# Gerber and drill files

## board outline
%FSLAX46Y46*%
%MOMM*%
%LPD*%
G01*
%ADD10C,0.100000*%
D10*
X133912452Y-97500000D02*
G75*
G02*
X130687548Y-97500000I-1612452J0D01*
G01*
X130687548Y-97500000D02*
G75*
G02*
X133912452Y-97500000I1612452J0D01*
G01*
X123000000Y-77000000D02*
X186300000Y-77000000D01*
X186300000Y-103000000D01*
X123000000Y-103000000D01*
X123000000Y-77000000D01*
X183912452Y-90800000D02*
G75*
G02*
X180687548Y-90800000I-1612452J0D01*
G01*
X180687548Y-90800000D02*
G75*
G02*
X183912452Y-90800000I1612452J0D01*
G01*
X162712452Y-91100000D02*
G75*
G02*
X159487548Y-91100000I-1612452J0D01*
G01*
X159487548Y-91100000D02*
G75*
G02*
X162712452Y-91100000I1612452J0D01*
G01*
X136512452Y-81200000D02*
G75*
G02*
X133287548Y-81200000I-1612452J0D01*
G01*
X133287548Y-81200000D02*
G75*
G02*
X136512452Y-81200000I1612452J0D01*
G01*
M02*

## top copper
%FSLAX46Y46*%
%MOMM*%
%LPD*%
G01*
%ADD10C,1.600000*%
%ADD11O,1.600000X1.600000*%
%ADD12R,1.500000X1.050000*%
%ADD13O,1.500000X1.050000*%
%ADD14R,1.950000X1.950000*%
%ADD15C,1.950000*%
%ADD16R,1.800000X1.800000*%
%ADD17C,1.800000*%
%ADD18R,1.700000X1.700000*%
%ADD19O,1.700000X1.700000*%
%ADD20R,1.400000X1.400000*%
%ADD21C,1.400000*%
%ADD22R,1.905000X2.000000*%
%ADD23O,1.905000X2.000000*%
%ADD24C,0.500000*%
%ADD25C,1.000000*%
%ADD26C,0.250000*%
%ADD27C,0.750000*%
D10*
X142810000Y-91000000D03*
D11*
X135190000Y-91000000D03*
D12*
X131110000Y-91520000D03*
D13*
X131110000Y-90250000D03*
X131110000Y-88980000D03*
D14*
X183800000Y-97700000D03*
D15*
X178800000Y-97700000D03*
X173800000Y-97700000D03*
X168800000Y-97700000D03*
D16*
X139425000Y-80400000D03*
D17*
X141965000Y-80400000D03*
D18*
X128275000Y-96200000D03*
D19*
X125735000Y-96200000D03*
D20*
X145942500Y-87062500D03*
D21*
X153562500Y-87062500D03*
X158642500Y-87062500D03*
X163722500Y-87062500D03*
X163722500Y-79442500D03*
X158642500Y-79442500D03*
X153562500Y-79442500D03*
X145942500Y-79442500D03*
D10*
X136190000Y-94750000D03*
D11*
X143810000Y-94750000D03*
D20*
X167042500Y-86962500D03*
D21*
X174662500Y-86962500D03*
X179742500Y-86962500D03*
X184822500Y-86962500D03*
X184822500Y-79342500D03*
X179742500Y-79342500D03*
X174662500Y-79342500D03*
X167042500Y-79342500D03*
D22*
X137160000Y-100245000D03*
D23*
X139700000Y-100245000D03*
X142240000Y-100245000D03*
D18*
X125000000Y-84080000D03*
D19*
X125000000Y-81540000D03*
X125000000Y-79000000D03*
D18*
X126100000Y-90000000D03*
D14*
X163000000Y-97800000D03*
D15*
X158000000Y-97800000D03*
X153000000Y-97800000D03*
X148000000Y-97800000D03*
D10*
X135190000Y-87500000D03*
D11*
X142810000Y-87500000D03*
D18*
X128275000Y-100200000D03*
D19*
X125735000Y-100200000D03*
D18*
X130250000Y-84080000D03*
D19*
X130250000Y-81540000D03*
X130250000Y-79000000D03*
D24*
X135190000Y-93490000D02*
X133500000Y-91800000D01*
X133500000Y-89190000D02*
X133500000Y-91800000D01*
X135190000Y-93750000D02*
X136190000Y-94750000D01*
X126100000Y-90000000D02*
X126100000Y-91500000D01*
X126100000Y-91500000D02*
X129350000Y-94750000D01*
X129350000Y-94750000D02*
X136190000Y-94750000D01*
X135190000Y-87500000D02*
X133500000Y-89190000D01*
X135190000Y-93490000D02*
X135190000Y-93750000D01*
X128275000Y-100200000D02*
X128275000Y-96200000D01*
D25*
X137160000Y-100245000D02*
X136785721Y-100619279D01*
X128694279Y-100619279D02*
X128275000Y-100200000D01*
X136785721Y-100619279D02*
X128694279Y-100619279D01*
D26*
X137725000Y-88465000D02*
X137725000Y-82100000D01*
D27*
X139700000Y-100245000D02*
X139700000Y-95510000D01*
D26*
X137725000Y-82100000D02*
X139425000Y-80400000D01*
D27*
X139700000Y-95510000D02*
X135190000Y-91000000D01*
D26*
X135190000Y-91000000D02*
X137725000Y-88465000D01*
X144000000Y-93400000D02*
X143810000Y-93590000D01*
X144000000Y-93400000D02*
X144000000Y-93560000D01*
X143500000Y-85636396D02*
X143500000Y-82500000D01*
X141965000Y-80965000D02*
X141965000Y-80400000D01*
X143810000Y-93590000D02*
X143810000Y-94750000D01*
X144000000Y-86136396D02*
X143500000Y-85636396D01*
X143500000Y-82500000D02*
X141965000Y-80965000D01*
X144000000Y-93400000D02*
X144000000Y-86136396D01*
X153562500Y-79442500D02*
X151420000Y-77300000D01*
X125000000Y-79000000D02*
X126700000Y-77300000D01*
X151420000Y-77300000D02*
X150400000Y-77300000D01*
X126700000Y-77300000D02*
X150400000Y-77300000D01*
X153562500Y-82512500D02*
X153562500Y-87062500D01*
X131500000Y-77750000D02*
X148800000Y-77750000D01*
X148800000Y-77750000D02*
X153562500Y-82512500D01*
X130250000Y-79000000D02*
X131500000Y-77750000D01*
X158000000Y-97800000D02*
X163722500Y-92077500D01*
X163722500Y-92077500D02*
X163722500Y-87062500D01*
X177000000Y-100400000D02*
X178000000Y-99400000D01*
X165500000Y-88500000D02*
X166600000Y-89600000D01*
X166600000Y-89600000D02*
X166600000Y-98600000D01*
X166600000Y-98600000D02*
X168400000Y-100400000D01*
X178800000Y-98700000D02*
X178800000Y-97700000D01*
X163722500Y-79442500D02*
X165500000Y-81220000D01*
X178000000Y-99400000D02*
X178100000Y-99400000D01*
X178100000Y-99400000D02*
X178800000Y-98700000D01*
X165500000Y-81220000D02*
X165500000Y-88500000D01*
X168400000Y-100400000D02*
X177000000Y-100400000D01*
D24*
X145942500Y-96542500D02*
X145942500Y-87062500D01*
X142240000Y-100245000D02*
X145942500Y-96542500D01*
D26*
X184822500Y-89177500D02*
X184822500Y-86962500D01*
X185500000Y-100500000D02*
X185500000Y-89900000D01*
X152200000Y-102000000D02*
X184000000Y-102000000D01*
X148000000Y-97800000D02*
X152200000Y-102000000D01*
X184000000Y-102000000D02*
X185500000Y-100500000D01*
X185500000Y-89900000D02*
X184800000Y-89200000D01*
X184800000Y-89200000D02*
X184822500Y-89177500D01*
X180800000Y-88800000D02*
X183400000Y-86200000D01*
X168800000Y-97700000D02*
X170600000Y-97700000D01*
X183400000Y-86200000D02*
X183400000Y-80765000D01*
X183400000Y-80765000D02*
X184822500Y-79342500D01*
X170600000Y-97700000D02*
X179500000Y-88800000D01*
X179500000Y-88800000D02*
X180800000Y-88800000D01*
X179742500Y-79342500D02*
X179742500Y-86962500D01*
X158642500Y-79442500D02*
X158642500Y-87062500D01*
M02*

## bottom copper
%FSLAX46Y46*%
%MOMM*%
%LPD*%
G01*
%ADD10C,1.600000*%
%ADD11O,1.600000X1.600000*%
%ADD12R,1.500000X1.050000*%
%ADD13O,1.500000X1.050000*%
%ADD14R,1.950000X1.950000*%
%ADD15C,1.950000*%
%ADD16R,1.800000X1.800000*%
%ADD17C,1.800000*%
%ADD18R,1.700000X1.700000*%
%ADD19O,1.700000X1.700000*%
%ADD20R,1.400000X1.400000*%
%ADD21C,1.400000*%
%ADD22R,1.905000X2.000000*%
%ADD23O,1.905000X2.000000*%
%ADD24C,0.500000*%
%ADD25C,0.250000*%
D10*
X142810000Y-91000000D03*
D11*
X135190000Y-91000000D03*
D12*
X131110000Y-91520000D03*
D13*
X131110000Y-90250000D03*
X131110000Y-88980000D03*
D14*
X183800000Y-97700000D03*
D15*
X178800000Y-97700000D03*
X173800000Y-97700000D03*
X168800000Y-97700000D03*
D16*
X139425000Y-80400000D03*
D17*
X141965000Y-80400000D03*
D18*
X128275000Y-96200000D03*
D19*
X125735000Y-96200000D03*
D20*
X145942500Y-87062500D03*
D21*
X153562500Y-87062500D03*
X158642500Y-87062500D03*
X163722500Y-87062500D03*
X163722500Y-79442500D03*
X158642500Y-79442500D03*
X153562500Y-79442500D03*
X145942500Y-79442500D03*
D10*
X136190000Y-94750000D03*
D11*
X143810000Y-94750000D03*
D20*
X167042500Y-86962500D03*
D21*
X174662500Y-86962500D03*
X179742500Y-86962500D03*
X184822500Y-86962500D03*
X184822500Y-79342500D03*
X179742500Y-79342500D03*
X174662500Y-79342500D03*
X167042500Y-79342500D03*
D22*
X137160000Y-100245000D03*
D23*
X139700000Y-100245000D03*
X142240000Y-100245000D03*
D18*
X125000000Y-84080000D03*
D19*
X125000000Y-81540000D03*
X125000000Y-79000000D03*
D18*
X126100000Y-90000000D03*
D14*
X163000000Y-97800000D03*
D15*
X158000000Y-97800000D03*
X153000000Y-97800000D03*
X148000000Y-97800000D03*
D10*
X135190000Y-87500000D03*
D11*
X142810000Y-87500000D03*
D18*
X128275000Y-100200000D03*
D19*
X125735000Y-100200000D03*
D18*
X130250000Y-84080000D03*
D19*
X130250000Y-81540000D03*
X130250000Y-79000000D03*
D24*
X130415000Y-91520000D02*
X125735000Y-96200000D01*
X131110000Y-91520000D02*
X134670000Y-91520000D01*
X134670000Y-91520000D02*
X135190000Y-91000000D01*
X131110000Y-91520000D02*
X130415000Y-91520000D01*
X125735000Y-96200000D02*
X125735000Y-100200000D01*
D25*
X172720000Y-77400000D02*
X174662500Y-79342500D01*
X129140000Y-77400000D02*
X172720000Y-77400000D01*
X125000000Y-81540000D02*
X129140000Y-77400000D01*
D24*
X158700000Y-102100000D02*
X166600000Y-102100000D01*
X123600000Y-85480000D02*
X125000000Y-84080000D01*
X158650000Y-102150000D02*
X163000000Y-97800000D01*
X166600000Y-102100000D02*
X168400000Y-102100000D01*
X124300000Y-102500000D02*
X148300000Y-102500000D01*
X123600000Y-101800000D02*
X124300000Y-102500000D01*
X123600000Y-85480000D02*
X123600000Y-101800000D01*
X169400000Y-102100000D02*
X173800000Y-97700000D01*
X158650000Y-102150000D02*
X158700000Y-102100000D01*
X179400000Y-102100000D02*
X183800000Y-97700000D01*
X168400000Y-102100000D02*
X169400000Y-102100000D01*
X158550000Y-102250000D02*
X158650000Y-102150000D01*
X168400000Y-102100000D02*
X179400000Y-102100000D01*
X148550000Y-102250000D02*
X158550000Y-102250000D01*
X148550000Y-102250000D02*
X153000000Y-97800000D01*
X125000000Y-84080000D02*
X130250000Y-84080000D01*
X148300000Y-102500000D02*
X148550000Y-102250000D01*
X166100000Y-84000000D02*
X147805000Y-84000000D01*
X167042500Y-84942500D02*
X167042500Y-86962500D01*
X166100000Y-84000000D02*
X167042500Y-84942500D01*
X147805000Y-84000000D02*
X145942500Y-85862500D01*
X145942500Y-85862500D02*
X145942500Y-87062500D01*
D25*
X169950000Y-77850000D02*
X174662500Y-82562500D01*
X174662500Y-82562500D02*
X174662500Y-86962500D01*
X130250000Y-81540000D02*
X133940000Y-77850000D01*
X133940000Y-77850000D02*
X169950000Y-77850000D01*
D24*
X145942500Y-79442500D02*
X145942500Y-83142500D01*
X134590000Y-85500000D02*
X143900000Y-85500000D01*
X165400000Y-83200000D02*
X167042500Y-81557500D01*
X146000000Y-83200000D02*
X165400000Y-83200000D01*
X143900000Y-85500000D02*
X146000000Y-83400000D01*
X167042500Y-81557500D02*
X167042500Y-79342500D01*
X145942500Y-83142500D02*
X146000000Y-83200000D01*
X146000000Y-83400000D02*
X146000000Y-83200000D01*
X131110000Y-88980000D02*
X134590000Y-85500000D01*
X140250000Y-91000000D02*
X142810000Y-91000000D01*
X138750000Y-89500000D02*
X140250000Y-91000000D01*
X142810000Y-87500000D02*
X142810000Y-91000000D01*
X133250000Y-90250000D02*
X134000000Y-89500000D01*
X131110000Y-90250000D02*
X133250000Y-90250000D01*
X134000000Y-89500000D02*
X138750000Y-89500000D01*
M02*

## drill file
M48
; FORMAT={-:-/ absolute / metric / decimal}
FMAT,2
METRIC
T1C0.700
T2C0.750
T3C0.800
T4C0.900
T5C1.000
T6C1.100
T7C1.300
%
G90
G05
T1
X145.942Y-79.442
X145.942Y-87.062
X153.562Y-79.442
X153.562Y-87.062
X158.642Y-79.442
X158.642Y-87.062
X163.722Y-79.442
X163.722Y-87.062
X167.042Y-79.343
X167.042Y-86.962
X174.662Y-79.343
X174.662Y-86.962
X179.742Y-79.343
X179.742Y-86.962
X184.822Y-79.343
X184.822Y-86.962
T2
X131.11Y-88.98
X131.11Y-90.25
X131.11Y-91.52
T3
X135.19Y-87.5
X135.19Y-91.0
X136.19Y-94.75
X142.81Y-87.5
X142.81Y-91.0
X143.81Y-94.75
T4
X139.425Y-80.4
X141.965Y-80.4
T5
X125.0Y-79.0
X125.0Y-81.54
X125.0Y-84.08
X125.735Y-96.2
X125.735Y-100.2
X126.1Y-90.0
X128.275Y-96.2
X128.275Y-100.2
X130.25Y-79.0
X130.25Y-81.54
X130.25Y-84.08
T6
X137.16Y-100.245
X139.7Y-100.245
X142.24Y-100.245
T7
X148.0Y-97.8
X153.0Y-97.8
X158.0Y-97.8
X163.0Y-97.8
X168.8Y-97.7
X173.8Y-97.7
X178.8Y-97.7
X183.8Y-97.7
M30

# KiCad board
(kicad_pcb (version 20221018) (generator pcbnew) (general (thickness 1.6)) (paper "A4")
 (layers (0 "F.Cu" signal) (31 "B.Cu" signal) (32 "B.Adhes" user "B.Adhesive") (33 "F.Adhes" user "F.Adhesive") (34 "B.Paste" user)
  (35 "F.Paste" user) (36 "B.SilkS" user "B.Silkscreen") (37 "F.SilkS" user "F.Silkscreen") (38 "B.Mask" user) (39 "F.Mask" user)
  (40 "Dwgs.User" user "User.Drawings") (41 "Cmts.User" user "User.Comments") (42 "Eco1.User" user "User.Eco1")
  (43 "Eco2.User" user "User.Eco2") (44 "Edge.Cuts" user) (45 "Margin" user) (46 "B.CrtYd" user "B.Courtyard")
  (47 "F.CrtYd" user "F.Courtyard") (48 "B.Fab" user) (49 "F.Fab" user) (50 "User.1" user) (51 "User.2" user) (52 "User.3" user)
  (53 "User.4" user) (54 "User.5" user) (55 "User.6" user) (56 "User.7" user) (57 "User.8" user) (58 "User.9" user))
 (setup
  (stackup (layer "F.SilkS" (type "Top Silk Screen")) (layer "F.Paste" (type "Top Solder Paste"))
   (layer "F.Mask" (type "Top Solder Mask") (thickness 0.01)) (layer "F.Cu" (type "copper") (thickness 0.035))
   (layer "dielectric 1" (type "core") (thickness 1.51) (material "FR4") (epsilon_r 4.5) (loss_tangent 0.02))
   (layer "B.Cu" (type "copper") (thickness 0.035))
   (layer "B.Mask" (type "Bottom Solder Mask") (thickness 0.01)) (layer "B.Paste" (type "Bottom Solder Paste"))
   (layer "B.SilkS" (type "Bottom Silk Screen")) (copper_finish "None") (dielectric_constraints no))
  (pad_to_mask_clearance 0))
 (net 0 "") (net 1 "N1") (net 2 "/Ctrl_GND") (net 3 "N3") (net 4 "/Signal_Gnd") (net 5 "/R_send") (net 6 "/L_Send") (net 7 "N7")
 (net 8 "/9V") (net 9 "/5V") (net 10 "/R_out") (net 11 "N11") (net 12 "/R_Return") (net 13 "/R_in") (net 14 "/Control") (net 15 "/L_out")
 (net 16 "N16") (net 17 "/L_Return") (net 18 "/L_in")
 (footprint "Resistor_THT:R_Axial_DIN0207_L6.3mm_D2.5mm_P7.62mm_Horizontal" (layer "F.Cu") (at 142.81 91 180)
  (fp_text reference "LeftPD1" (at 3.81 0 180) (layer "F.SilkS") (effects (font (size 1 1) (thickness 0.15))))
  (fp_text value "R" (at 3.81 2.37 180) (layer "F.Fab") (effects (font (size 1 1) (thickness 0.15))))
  (pad "1" thru_hole circle (at 0 0 180) (size 1.6 1.6) (drill 0.8) (layers "*.Cu" "*.Mask") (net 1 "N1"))
  (pad "2" thru_hole oval (at 7.62 0 180) (size 1.6 1.6) (drill 0.8) (layers "*.Cu" "*.Mask") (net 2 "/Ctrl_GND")))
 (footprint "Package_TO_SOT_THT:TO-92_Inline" (layer "F.Cu") (at 131.11 91.52 90)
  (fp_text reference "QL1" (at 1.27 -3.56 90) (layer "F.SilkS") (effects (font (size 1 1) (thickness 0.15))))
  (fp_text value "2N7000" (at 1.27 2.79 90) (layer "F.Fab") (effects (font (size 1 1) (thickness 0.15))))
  (pad "1" thru_hole rect (at 0 0 90) (size 1.05 1.5) (drill 0.75) (layers "*.Cu" "*.Mask") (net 2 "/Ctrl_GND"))
  (pad "2" thru_hole oval (at 1.27 0 90) (size 1.05 1.5) (drill 0.75) (layers "*.Cu" "*.Mask") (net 1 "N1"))
  (pad "3" thru_hole oval (at 2.54 0 90) (size 1.05 1.5) (drill 0.75) (layers "*.Cu" "*.Mask") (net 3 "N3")))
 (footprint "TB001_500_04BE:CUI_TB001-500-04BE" (layer "F.Cu") (at 183.8 97.7 180)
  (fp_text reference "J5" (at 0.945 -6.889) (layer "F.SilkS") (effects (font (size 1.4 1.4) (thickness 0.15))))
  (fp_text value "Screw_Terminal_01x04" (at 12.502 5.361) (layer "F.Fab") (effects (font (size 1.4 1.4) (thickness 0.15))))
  (pad "1" thru_hole rect (at 0 0 180) (size 1.95 1.95) (drill 1.3) (layers "*.Cu" "*.Mask") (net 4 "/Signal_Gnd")
   (solder_mask_margin 0.102))
  (pad "2" thru_hole circle (at 5 0 180) (size 1.95 1.95) (drill 1.3) (layers "*.Cu" "*.Mask") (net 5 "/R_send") (solder_mask_margin 0.102))
  (pad "3" thru_hole circle (at 10 0 180) (size 1.95 1.95) (drill 1.3) (layers "*.Cu" "*.Mask") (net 4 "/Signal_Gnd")
   (solder_mask_margin 0.102))
  (pad "4" thru_hole circle (at 15 0 180) (size 1.95 1.95) (drill 1.3) (layers "*.Cu" "*.Mask") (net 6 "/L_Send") (solder_mask_margin 0.102)))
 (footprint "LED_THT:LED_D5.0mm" (layer "F.Cu") (at 139.425 80.4)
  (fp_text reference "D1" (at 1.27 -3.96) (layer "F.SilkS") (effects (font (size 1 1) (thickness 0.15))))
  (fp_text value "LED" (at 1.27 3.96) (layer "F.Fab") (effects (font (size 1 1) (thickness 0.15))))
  (pad "1" thru_hole rect (at 0 0) (size 1.8 1.8) (drill 0.9) (layers "*.Cu" "*.Mask") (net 2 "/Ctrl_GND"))
  (pad "2" thru_hole circle (at 2.54 0) (size 1.8 1.8) (drill 0.9) (layers "*.Cu" "*.Mask") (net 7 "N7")))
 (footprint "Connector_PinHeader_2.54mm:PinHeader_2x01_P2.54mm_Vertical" (layer "F.Cu") (at 128.275 96.2 180)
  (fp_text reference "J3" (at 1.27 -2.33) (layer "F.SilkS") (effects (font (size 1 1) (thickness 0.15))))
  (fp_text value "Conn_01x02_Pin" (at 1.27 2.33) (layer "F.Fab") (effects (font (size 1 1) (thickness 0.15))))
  (pad "1" thru_hole rect (at 0 0 180) (size 1.7 1.7) (drill 1) (layers "*.Cu" "*.Mask") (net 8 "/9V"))
  (pad "2" thru_hole oval (at 2.54 0 180) (size 1.7 1.7) (drill 1) (layers "*.Cu" "*.Mask") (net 2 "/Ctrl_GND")))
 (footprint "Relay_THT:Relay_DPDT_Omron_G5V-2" (layer "F.Cu") (at 145.9425 87.0625 90)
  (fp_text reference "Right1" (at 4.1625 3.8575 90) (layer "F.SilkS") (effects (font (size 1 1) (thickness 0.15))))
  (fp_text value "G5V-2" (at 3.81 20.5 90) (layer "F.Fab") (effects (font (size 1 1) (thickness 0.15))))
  (pad "1" thru_hole rect (at 0 0 90) (size 1.4 1.4) (drill 0.7) (layers "*.Cu" "*.Mask") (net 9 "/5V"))
  (pad "4" thru_hole circle (at 0 7.62 90) (size 1.4 1.4) (drill 0.7) (layers "*.Cu" "*.Mask") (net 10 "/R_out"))
  (pad "6" thru_hole circle (at 0 12.7 90) (size 1.4 1.4) (drill 0.7) (layers "*.Cu" "*.Mask") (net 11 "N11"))
  (pad "8" thru_hole circle (at 0 17.78 90) (size 1.4 1.4) (drill 0.7) (layers "*.Cu" "*.Mask") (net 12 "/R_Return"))
  (pad "9" thru_hole circle (at 7.62 17.78 90) (size 1.4 1.4) (drill 0.7) (layers "*.Cu" "*.Mask") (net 5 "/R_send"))
  (pad "11" thru_hole circle (at 7.62 12.7 90) (size 1.4 1.4) (drill 0.7) (layers "*.Cu" "*.Mask") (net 11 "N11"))
  (pad "13" thru_hole circle (at 7.62 7.62 90) (size 1.4 1.4) (drill 0.7) (layers "*.Cu" "*.Mask") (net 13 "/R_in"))
  (pad "16" thru_hole circle (at 7.62 0 90) (size 1.4 1.4) (drill 0.7) (layers "*.Cu" "*.Mask") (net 3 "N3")))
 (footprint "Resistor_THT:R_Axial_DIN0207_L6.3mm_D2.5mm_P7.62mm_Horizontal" (layer "F.Cu") (at 136.19 94.75)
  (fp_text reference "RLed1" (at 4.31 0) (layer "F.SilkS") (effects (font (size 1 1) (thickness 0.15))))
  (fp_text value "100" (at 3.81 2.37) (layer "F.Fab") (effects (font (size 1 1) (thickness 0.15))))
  (pad "1" thru_hole circle (at 0 0) (size 1.6 1.6) (drill 0.8) (layers "*.Cu" "*.Mask") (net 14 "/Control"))
  (pad "2" thru_hole oval (at 7.62 0) (size 1.6 1.6) (drill 0.8) (layers "*.Cu" "*.Mask") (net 7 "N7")))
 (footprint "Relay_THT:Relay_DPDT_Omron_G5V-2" (layer "F.Cu") (at 167.0425 86.9625 90)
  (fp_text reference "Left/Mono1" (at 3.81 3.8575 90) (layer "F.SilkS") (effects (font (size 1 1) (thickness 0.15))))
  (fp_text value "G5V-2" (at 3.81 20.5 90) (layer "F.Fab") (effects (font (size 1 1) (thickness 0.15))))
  (pad "1" thru_hole rect (at 0 0 90) (size 1.4 1.4) (drill 0.7) (layers "*.Cu" "*.Mask") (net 9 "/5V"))
  (pad "4" thru_hole circle (at 0 7.62 90) (size 1.4 1.4) (drill 0.7) (layers "*.Cu" "*.Mask") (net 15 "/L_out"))
  (pad "6" thru_hole circle (at 0 12.7 90) (size 1.4 1.4) (drill 0.7) (layers "*.Cu" "*.Mask") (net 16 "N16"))
  (pad "8" thru_hole circle (at 0 17.78 90) (size 1.4 1.4) (drill 0.7) (layers "*.Cu" "*.Mask") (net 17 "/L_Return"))
  (pad "9" thru_hole circle (at 7.62 17.78 90) (size 1.4 1.4) (drill 0.7) (layers "*.Cu" "*.Mask") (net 6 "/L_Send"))
  (pad "11" thru_hole circle (at 7.62 12.7 90) (size 1.4 1.4) (drill 0.7) (layers "*.Cu" "*.Mask") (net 16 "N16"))
  (pad "13" thru_hole circle (at 7.62 7.62 90) (size 1.4 1.4) (drill 0.7) (layers "*.Cu" "*.Mask") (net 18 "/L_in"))
  (pad "16" thru_hole circle (at 7.62 0 90) (size 1.4 1.4) (drill 0.7) (layers "*.Cu" "*.Mask") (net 3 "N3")))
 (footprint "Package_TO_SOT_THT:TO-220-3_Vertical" (layer "F.Cu") (at 137.16 100.245)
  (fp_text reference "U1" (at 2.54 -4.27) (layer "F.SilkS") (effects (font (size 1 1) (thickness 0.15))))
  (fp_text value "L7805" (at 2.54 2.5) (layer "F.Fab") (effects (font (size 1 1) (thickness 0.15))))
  (pad "1" thru_hole rect (at 0 0) (size 1.905 2) (drill 1.1) (layers "*.Cu" "*.Mask") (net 8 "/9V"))
  (pad "2" thru_hole oval (at 2.54 0) (size 1.905 2) (drill 1.1) (layers "*.Cu" "*.Mask") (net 2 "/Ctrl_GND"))
  (pad "3" thru_hole oval (at 5.08 0) (size 1.905 2) (drill 1.1) (layers "*.Cu" "*.Mask") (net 9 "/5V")))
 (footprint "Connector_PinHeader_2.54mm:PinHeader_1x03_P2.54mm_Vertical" (layer "F.Cu") (at 125 84.08 180)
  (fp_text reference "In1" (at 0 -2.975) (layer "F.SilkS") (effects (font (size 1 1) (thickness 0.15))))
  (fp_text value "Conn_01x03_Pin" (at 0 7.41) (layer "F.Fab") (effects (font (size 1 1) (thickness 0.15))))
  (pad "1" thru_hole rect (at 0 0 180) (size 1.7 1.7) (drill 1) (layers "*.Cu" "*.Mask") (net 4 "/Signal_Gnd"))
  (pad "2" thru_hole oval (at 0 2.54 180) (size 1.7 1.7) (drill 1) (layers "*.Cu" "*.Mask") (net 18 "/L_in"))
  (pad "3" thru_hole oval (at 0 5.08 180) (size 1.7 1.7) (drill 1) (layers "*.Cu" "*.Mask") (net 13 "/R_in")))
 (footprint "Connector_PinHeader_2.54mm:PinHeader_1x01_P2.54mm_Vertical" (layer "F.Cu") (at 126.1 90 90)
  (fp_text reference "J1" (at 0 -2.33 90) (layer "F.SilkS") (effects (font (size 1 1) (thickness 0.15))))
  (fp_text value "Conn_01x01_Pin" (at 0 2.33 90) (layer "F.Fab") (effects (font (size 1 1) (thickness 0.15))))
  (pad "1" thru_hole rect (at 0 0 90) (size 1.7 1.7) (drill 1) (layers "*.Cu" "*.Mask") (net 14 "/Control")))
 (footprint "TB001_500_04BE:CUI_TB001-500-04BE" (layer "F.Cu") (at 163 97.8 180)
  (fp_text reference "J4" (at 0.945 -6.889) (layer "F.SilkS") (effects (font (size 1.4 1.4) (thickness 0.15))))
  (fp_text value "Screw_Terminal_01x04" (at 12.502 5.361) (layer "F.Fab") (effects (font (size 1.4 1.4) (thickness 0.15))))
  (pad "1" thru_hole rect (at 0 0 180) (size 1.95 1.95) (drill 1.3) (layers "*.Cu" "*.Mask") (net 4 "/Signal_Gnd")
   (solder_mask_margin 0.102))
  (pad "2" thru_hole circle (at 5 0 180) (size 1.95 1.95) (drill 1.3) (layers "*.Cu" "*.Mask") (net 12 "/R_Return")
   (solder_mask_margin 0.102))
  (pad "3" thru_hole circle (at 10 0 180) (size 1.95 1.95) (drill 1.3) (layers "*.Cu" "*.Mask") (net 4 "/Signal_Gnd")
   (solder_mask_margin 0.102))
  (pad "4" thru_hole circle (at 15 0 180) (size 1.95 1.95) (drill 1.3) (layers "*.Cu" "*.Mask") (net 17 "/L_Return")
   (solder_mask_margin 0.102)))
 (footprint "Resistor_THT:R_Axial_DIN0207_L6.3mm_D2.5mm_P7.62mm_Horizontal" (layer "F.Cu") (at 135.19 87.5)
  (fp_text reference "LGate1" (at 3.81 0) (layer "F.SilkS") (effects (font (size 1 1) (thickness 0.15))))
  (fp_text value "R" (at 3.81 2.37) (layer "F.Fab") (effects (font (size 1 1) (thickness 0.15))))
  (pad "1" thru_hole circle (at 0 0) (size 1.6 1.6) (drill 0.8) (layers "*.Cu" "*.Mask") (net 14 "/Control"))
  (pad "2" thru_hole oval (at 7.62 0) (size 1.6 1.6) (drill 0.8) (layers "*.Cu" "*.Mask") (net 1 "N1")))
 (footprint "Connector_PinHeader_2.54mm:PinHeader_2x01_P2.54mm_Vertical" (layer "F.Cu") (at 128.275 100.2 180)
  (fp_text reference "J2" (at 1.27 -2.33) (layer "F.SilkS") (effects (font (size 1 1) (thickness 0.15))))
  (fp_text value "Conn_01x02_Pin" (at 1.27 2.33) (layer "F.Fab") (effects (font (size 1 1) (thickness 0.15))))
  (pad "1" thru_hole rect (at 0 0 180) (size 1.7 1.7) (drill 1) (layers "*.Cu" "*.Mask") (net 8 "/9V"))
  (pad "2" thru_hole oval (at 2.54 0 180) (size 1.7 1.7) (drill 1) (layers "*.Cu" "*.Mask") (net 2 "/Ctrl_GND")))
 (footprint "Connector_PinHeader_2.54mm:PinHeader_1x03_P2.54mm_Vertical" (layer "F.Cu") (at 130.25 84.08 180)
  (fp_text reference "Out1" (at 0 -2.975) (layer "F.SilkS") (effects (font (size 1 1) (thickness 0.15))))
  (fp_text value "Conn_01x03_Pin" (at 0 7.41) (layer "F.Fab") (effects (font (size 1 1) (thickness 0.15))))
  (pad "1" thru_hole rect (at 0 0 180) (size 1.7 1.7) (drill 1) (layers "*.Cu" "*.Mask") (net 4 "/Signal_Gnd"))
  (pad "2" thru_hole oval (at 0 2.54 180) (size 1.7 1.7) (drill 1) (layers "*.Cu" "*.Mask") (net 15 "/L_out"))
  (pad "3" thru_hole oval (at 0 5.08 180) (size 1.7 1.7) (drill 1) (layers "*.Cu" "*.Mask") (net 10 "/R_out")))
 (gr_circle (center 132.3 97.5) (end 132.1 95.9) (stroke (width 0.1) (type default)) (fill none) (layer "Edge.Cuts"))
 (gr_rect (start 123 77) (end 186.3 103) (stroke (width 0.1) (type default)) (fill none) (layer "Edge.Cuts"))
 (gr_circle (center 182.3 90.8) (end 182.1 89.2) (stroke (width 0.1) (type default)) (fill none) (layer "Edge.Cuts"))
 (gr_circle (center 161.1 91.1) (end 160.9 89.5) (stroke (width 0.1) (type default)) (fill none) (layer "Edge.Cuts"))
 (gr_circle (center 134.9 81.2) (end 134.7 79.6) (stroke (width 0.1) (type default)) (fill none) (layer "Edge.Cuts"))
 (segment (start 135.19 93.49) (end 133.5 91.8) (width 0.5) (layer "F.Cu") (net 14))
 (segment (start 133.5 89.19) (end 133.5 91.8) (width 0.5) (layer "F.Cu") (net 14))
 (segment (start 135.19 93.75) (end 136.19 94.75) (width 0.5) (layer "F.Cu") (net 14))
 (segment (start 126.1 90) (end 126.1 91.5) (width 0.5) (layer "F.Cu") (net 14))
 (segment (start 126.1 91.5) (end 129.35 94.75) (width 0.5) (layer "F.Cu") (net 14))
 (segment (start 129.35 94.75) (end 136.19 94.75) (width 0.5) (layer "F.Cu") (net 14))
 (segment (start 135.19 87.5) (end 133.5 89.19) (width 0.5) (layer "F.Cu") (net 14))
 (segment (start 135.19 93.49) (end 135.19 93.75) (width 0.5) (layer "F.Cu") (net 14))
 (segment (start 128.275 100.2) (end 128.275 96.2) (width 0.5) (layer "F.Cu") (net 8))
 (segment (start 137.16 100.245) (end 136.785721 100.619279) (width 1) (layer "F.Cu") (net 8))
 (segment (start 128.694279 100.619279) (end 128.275 100.2) (width 1) (layer "F.Cu") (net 8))
 (segment (start 136.785721 100.619279) (end 128.694279 100.619279) (width 1) (layer "F.Cu") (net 8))
 (segment (start 137.725 88.465) (end 137.725 82.1) (width 0.25) (layer "F.Cu") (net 2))
 (segment (start 139.7 100.245) (end 139.7 95.51) (width 0.75) (layer "F.Cu") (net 2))
 (segment (start 137.725 82.1) (end 139.425 80.4) (width 0.25) (layer "F.Cu") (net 2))
 (segment (start 139.7 95.51) (end 135.19 91) (width 0.75) (layer "F.Cu") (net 2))
 (segment (start 135.19 91) (end 137.725 88.465) (width 0.25) (layer "F.Cu") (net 2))
 (segment (start 130.415 91.52) (end 125.735 96.2) (width 0.5) (layer "B.Cu") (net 2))
 (segment (start 131.11 91.52) (end 134.67 91.52) (width 0.5) (layer "B.Cu") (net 2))
 (segment (start 134.67 91.52) (end 135.19 91) (width 0.5) (layer "B.Cu") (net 2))
 (segment (start 131.11 91.52) (end 130.415 91.52) (width 0.5) (layer "B.Cu") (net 2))
 (segment (start 125.735 96.2) (end 125.735 100.2) (width 0.5) (layer "B.Cu") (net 2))
 (segment (start 144 93.4) (end 143.81 93.59) (width 0.25) (layer "F.Cu") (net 7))
 (segment (start 144 93.4) (end 144 93.56) (width 0.25) (layer "F.Cu") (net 7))
 (segment (start 143.5 85.636396) (end 143.5 82.5) (width 0.25) (layer "F.Cu") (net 7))
 (segment (start 141.965 80.965) (end 141.965 80.4) (width 0.25) (layer "F.Cu") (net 7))
 (segment (start 143.81 93.59) (end 143.81 94.75) (width 0.25) (layer "F.Cu") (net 7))
 (segment (start 144 86.136396) (end 143.5 85.636396) (width 0.25) (layer "F.Cu") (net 7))
 (segment (start 143.5 82.5) (end 141.965 80.965) (width 0.25) (layer "F.Cu") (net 7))
 (segment (start 144 93.4) (end 144 86.136396) (width 0.25) (layer "F.Cu") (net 7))
 (segment (start 153.5625 79.4425) (end 151.42 77.3) (width 0.25) (layer "F.Cu") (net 13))
 (segment (start 125 79) (end 126.7 77.3) (width 0.25) (layer "F.Cu") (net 13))
 (segment (start 151.42 77.3) (end 150.4 77.3) (width 0.25) (layer "F.Cu") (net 13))
 (segment (start 126.7 77.3) (end 150.4 77.3) (width 0.25) (layer "F.Cu") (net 13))
 (segment (start 172.72 77.4) (end 174.6625 79.3425) (width 0.25) (layer "B.Cu") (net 18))
 (segment (start 129.14 77.4) (end 172.72 77.4) (width 0.25) (layer "B.Cu") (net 18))
 (segment (start 125 81.54) (end 129.14 77.4) (width 0.25) (layer "B.Cu") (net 18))
 (segment (start 158.7 102.1) (end 166.6 102.1) (width 0.5) (layer "B.Cu") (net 4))
 (segment (start 123.6 85.48) (end 125 84.08) (width 0.5) (layer "B.Cu") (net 4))
 (segment (start 158.65 102.15) (end 163 97.8) (width 0.5) (layer "B.Cu") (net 4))
 (segment (start 166.6 102.1) (end 168.4 102.1) (width 0.5) (layer "B.Cu") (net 4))
 (segment (start 124.3 102.5) (end 148.3 102.5) (width 0.5) (layer "B.Cu") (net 4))
 (segment (start 123.6 101.8) (end 124.3 102.5) (width 0.5) (layer "B.Cu") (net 4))
 (segment (start 123.6 85.48) (end 123.6 101.8) (width 0.5) (layer "B.Cu") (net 4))
 (segment (start 169.4 102.1) (end 173.8 97.7) (width 0.5) (layer "B.Cu") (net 4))
 (segment (start 158.65 102.15) (end 158.7 102.1) (width 0.5) (layer "B.Cu") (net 4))
 (segment (start 179.4 102.1) (end 183.8 97.7) (width 0.5) (layer "B.Cu") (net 4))
 (segment (start 168.4 102.1) (end 169.4 102.1) (width 0.5) (layer "B.Cu") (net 4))
 (segment (start 158.55 102.25) (end 158.65 102.15) (width 0.5) (layer "B.Cu") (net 4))
 (segment (start 168.4 102.1) (end 179.4 102.1) (width 0.5) (layer "B.Cu") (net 4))
 (segment (start 148.55 102.25) (end 158.55 102.25) (width 0.5) (layer "B.Cu") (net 4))
 (segment (start 148.55 102.25) (end 153 97.8) (width 0.5) (layer "B.Cu") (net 4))
 (segment (start 125 84.08) (end 130.25 84.08) (width 0.5) (layer "B.Cu") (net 4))
 (segment (start 148.3 102.5) (end 148.55 102.25) (width 0.5) (layer "B.Cu") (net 4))
 (segment (start 153.5625 82.5125) (end 153.5625 87.0625) (width 0.25) (layer "F.Cu") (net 10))
 (segment (start 131.5 77.75) (end 148.8 77.75) (width 0.25) (layer "F.Cu") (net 10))
 (segment (start 148.8 77.75) (end 153.5625 82.5125) (width 0.25) (layer "F.Cu") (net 10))
 (segment (start 130.25 79) (end 131.5 77.75) (width 0.25) (layer "F.Cu") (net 10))
 (segment (start 158 97.8) (end 163.7225 92.0775) (width 0.25) (layer "F.Cu") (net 12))
 (segment (start 163.7225 92.0775) (end 163.7225 87.0625) (width 0.25) (layer "F.Cu") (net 12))
 (segment (start 177 100.4) (end 178 99.4) (width 0.25) (layer "F.Cu") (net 5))
 (segment (start 165.5 88.5) (end 166.6 89.6) (width 0.25) (layer "F.Cu") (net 5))
 (segment (start 166.6 89.6) (end 166.6 98.6) (width 0.25) (layer "F.Cu") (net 5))
 (segment (start 166.6 98.6) (end 168.4 100.4) (width 0.25) (layer "F.Cu") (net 5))
 (segment (start 178.8 98.7) (end 178.8 97.7) (width 0.25) (layer "F.Cu") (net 5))
 (segment (start 163.7225 79.4425) (end 165.5 81.22) (width 0.25) (layer "F.Cu") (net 5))
 (segment (start 178 99.4) (end 178.1 99.4) (width 0.25) (layer "F.Cu") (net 5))
 (segment (start 178.1 99.4) (end 178.8 98.7) (width 0.25) (layer "F.Cu") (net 5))
 (segment (start 165.5 81.22) (end 165.5 88.5) (width 0.25) (layer "F.Cu") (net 5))
 (segment (start 168.4 100.4) (end 177 100.4) (width 0.25) (layer "F.Cu") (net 5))
 (segment (start 145.9425 96.5425) (end 145.9425 87.0625) (width 0.5) (layer "F.Cu") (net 9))
 (segment (start 142.24 100.245) (end 145.9425 96.5425) (width 0.5) (layer "F.Cu") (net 9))
 (segment (start 166.1 84) (end 147.805 84) (width 0.5) (layer "B.Cu") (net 9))
 (segment (start 167.0425 84.9425) (end 167.0425 86.9625) (width 0.5) (layer "B.Cu") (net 9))
 (segment (start 166.1 84) (end 167.0425 84.9425) (width 0.5) (layer "B.Cu") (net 9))
 (segment (start 147.805 84) (end 145.9425 85.8625) (width 0.5) (layer "B.Cu") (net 9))
 (segment (start 145.9425 85.8625) (end 145.9425 87.0625) (width 0.5) (layer "B.Cu") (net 9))
 (segment (start 169.95 77.85) (end 174.6625 82.5625) (width 0.25) (layer "B.Cu") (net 15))
 (segment (start 174.6625 82.5625) (end 174.6625 86.9625) (width 0.25) (layer "B.Cu") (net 15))
 (segment (start 130.25 81.54) (end 133.94 77.85) (width 0.25) (layer "B.Cu") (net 15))
 (segment (start 133.94 77.85) (end 169.95 77.85) (width 0.25) (layer "B.Cu") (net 15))
 (segment (start 184.8225 89.1775) (end 184.8225 86.9625) (width 0.25) (layer "F.Cu") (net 17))
 (segment (start 185.5 100.5) (end 185.5 89.9) (width 0.25) (layer "F.Cu") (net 17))
 (segment (start 152.2 102) (end 184 102) (width 0.25) (layer "F.Cu") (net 17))
 (segment (start 148 97.8) (end 152.2 102) (width 0.25) (layer "F.Cu") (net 17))
 (segment (start 184 102) (end 185.5 100.5) (width 0.25) (layer "F.Cu") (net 17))
 (segment (start 185.5 89.9) (end 184.8 89.2) (width 0.25) (layer "F.Cu") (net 17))
 (segment (start 184.8 89.2) (end 184.8225 89.1775) (width 0.25) (layer "F.Cu") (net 17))
 (segment (start 180.8 88.8) (end 183.4 86.2) (width 0.25) (layer "F.Cu") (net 6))
 (segment (start 168.8 97.7) (end 170.6 97.7) (width 0.25) (layer "F.Cu") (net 6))
 (segment (start 183.4 86.2) (end 183.4 80.765) (width 0.25) (layer "F.Cu") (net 6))
 (segment (start 183.4 80.765) (end 184.8225 79.3425) (width 0.25) (layer "F.Cu") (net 6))
 (segment (start 170.6 97.7) (end 179.5 88.8) (width 0.25) (layer "F.Cu") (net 6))
 (segment (start 179.5 88.8) (end 180.8 88.8) (width 0.25) (layer "F.Cu") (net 6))
 (segment (start 179.7425 79.3425) (end 179.7425 86.9625) (width 0.25) (layer "F.Cu") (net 16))
 (segment (start 158.6425 79.4425) (end 158.6425 87.0625) (width 0.25) (layer "F.Cu") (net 11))
 (segment (start 145.9425 79.4425) (end 145.9425 83.1425) (width 0.5) (layer "B.Cu") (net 3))
 (segment (start 134.59 85.5) (end 143.9 85.5) (width 0.5) (layer "B.Cu") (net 3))
 (segment (start 165.4 83.2) (end 167.0425 81.5575) (width 0.5) (layer "B.Cu") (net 3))
 (segment (start 146 83.2) (end 165.4 83.2) (width 0.5) (layer "B.Cu") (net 3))
 (segment (start 143.9 85.5) (end 146 83.4) (width 0.5) (layer "B.Cu") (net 3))
 (segment (start 167.0425 81.5575) (end 167.0425 79.3425) (width 0.5) (layer "B.Cu") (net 3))
 (segment (start 145.9425 83.1425) (end 146 83.2) (width 0.5) (layer "B.Cu") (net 3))
 (segment (start 146 83.4) (end 146 83.2) (width 0.5) (layer "B.Cu") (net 3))
 (segment (start 131.11 88.98) (end 134.59 85.5) (width 0.5) (layer "B.Cu") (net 3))
 (segment (start 140.25 91) (end 142.81 91) (width 0.5) (layer "B.Cu") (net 1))
 (segment (start 138.75 89.5) (end 140.25 91) (width 0.5) (layer "B.Cu") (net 1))
 (segment (start 142.81 87.5) (end 142.81 91) (width 0.5) (layer "B.Cu") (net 1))
 (segment (start 133.25 90.25) (end 134 89.5) (width 0.5) (layer "B.Cu") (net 1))
 (segment (start 131.11 90.25) (end 133.25 90.25) (width 0.5) (layer "B.Cu") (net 1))
 (segment (start 134 89.5) (end 138.75 89.5) (width 0.5) (layer "B.Cu") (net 1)))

